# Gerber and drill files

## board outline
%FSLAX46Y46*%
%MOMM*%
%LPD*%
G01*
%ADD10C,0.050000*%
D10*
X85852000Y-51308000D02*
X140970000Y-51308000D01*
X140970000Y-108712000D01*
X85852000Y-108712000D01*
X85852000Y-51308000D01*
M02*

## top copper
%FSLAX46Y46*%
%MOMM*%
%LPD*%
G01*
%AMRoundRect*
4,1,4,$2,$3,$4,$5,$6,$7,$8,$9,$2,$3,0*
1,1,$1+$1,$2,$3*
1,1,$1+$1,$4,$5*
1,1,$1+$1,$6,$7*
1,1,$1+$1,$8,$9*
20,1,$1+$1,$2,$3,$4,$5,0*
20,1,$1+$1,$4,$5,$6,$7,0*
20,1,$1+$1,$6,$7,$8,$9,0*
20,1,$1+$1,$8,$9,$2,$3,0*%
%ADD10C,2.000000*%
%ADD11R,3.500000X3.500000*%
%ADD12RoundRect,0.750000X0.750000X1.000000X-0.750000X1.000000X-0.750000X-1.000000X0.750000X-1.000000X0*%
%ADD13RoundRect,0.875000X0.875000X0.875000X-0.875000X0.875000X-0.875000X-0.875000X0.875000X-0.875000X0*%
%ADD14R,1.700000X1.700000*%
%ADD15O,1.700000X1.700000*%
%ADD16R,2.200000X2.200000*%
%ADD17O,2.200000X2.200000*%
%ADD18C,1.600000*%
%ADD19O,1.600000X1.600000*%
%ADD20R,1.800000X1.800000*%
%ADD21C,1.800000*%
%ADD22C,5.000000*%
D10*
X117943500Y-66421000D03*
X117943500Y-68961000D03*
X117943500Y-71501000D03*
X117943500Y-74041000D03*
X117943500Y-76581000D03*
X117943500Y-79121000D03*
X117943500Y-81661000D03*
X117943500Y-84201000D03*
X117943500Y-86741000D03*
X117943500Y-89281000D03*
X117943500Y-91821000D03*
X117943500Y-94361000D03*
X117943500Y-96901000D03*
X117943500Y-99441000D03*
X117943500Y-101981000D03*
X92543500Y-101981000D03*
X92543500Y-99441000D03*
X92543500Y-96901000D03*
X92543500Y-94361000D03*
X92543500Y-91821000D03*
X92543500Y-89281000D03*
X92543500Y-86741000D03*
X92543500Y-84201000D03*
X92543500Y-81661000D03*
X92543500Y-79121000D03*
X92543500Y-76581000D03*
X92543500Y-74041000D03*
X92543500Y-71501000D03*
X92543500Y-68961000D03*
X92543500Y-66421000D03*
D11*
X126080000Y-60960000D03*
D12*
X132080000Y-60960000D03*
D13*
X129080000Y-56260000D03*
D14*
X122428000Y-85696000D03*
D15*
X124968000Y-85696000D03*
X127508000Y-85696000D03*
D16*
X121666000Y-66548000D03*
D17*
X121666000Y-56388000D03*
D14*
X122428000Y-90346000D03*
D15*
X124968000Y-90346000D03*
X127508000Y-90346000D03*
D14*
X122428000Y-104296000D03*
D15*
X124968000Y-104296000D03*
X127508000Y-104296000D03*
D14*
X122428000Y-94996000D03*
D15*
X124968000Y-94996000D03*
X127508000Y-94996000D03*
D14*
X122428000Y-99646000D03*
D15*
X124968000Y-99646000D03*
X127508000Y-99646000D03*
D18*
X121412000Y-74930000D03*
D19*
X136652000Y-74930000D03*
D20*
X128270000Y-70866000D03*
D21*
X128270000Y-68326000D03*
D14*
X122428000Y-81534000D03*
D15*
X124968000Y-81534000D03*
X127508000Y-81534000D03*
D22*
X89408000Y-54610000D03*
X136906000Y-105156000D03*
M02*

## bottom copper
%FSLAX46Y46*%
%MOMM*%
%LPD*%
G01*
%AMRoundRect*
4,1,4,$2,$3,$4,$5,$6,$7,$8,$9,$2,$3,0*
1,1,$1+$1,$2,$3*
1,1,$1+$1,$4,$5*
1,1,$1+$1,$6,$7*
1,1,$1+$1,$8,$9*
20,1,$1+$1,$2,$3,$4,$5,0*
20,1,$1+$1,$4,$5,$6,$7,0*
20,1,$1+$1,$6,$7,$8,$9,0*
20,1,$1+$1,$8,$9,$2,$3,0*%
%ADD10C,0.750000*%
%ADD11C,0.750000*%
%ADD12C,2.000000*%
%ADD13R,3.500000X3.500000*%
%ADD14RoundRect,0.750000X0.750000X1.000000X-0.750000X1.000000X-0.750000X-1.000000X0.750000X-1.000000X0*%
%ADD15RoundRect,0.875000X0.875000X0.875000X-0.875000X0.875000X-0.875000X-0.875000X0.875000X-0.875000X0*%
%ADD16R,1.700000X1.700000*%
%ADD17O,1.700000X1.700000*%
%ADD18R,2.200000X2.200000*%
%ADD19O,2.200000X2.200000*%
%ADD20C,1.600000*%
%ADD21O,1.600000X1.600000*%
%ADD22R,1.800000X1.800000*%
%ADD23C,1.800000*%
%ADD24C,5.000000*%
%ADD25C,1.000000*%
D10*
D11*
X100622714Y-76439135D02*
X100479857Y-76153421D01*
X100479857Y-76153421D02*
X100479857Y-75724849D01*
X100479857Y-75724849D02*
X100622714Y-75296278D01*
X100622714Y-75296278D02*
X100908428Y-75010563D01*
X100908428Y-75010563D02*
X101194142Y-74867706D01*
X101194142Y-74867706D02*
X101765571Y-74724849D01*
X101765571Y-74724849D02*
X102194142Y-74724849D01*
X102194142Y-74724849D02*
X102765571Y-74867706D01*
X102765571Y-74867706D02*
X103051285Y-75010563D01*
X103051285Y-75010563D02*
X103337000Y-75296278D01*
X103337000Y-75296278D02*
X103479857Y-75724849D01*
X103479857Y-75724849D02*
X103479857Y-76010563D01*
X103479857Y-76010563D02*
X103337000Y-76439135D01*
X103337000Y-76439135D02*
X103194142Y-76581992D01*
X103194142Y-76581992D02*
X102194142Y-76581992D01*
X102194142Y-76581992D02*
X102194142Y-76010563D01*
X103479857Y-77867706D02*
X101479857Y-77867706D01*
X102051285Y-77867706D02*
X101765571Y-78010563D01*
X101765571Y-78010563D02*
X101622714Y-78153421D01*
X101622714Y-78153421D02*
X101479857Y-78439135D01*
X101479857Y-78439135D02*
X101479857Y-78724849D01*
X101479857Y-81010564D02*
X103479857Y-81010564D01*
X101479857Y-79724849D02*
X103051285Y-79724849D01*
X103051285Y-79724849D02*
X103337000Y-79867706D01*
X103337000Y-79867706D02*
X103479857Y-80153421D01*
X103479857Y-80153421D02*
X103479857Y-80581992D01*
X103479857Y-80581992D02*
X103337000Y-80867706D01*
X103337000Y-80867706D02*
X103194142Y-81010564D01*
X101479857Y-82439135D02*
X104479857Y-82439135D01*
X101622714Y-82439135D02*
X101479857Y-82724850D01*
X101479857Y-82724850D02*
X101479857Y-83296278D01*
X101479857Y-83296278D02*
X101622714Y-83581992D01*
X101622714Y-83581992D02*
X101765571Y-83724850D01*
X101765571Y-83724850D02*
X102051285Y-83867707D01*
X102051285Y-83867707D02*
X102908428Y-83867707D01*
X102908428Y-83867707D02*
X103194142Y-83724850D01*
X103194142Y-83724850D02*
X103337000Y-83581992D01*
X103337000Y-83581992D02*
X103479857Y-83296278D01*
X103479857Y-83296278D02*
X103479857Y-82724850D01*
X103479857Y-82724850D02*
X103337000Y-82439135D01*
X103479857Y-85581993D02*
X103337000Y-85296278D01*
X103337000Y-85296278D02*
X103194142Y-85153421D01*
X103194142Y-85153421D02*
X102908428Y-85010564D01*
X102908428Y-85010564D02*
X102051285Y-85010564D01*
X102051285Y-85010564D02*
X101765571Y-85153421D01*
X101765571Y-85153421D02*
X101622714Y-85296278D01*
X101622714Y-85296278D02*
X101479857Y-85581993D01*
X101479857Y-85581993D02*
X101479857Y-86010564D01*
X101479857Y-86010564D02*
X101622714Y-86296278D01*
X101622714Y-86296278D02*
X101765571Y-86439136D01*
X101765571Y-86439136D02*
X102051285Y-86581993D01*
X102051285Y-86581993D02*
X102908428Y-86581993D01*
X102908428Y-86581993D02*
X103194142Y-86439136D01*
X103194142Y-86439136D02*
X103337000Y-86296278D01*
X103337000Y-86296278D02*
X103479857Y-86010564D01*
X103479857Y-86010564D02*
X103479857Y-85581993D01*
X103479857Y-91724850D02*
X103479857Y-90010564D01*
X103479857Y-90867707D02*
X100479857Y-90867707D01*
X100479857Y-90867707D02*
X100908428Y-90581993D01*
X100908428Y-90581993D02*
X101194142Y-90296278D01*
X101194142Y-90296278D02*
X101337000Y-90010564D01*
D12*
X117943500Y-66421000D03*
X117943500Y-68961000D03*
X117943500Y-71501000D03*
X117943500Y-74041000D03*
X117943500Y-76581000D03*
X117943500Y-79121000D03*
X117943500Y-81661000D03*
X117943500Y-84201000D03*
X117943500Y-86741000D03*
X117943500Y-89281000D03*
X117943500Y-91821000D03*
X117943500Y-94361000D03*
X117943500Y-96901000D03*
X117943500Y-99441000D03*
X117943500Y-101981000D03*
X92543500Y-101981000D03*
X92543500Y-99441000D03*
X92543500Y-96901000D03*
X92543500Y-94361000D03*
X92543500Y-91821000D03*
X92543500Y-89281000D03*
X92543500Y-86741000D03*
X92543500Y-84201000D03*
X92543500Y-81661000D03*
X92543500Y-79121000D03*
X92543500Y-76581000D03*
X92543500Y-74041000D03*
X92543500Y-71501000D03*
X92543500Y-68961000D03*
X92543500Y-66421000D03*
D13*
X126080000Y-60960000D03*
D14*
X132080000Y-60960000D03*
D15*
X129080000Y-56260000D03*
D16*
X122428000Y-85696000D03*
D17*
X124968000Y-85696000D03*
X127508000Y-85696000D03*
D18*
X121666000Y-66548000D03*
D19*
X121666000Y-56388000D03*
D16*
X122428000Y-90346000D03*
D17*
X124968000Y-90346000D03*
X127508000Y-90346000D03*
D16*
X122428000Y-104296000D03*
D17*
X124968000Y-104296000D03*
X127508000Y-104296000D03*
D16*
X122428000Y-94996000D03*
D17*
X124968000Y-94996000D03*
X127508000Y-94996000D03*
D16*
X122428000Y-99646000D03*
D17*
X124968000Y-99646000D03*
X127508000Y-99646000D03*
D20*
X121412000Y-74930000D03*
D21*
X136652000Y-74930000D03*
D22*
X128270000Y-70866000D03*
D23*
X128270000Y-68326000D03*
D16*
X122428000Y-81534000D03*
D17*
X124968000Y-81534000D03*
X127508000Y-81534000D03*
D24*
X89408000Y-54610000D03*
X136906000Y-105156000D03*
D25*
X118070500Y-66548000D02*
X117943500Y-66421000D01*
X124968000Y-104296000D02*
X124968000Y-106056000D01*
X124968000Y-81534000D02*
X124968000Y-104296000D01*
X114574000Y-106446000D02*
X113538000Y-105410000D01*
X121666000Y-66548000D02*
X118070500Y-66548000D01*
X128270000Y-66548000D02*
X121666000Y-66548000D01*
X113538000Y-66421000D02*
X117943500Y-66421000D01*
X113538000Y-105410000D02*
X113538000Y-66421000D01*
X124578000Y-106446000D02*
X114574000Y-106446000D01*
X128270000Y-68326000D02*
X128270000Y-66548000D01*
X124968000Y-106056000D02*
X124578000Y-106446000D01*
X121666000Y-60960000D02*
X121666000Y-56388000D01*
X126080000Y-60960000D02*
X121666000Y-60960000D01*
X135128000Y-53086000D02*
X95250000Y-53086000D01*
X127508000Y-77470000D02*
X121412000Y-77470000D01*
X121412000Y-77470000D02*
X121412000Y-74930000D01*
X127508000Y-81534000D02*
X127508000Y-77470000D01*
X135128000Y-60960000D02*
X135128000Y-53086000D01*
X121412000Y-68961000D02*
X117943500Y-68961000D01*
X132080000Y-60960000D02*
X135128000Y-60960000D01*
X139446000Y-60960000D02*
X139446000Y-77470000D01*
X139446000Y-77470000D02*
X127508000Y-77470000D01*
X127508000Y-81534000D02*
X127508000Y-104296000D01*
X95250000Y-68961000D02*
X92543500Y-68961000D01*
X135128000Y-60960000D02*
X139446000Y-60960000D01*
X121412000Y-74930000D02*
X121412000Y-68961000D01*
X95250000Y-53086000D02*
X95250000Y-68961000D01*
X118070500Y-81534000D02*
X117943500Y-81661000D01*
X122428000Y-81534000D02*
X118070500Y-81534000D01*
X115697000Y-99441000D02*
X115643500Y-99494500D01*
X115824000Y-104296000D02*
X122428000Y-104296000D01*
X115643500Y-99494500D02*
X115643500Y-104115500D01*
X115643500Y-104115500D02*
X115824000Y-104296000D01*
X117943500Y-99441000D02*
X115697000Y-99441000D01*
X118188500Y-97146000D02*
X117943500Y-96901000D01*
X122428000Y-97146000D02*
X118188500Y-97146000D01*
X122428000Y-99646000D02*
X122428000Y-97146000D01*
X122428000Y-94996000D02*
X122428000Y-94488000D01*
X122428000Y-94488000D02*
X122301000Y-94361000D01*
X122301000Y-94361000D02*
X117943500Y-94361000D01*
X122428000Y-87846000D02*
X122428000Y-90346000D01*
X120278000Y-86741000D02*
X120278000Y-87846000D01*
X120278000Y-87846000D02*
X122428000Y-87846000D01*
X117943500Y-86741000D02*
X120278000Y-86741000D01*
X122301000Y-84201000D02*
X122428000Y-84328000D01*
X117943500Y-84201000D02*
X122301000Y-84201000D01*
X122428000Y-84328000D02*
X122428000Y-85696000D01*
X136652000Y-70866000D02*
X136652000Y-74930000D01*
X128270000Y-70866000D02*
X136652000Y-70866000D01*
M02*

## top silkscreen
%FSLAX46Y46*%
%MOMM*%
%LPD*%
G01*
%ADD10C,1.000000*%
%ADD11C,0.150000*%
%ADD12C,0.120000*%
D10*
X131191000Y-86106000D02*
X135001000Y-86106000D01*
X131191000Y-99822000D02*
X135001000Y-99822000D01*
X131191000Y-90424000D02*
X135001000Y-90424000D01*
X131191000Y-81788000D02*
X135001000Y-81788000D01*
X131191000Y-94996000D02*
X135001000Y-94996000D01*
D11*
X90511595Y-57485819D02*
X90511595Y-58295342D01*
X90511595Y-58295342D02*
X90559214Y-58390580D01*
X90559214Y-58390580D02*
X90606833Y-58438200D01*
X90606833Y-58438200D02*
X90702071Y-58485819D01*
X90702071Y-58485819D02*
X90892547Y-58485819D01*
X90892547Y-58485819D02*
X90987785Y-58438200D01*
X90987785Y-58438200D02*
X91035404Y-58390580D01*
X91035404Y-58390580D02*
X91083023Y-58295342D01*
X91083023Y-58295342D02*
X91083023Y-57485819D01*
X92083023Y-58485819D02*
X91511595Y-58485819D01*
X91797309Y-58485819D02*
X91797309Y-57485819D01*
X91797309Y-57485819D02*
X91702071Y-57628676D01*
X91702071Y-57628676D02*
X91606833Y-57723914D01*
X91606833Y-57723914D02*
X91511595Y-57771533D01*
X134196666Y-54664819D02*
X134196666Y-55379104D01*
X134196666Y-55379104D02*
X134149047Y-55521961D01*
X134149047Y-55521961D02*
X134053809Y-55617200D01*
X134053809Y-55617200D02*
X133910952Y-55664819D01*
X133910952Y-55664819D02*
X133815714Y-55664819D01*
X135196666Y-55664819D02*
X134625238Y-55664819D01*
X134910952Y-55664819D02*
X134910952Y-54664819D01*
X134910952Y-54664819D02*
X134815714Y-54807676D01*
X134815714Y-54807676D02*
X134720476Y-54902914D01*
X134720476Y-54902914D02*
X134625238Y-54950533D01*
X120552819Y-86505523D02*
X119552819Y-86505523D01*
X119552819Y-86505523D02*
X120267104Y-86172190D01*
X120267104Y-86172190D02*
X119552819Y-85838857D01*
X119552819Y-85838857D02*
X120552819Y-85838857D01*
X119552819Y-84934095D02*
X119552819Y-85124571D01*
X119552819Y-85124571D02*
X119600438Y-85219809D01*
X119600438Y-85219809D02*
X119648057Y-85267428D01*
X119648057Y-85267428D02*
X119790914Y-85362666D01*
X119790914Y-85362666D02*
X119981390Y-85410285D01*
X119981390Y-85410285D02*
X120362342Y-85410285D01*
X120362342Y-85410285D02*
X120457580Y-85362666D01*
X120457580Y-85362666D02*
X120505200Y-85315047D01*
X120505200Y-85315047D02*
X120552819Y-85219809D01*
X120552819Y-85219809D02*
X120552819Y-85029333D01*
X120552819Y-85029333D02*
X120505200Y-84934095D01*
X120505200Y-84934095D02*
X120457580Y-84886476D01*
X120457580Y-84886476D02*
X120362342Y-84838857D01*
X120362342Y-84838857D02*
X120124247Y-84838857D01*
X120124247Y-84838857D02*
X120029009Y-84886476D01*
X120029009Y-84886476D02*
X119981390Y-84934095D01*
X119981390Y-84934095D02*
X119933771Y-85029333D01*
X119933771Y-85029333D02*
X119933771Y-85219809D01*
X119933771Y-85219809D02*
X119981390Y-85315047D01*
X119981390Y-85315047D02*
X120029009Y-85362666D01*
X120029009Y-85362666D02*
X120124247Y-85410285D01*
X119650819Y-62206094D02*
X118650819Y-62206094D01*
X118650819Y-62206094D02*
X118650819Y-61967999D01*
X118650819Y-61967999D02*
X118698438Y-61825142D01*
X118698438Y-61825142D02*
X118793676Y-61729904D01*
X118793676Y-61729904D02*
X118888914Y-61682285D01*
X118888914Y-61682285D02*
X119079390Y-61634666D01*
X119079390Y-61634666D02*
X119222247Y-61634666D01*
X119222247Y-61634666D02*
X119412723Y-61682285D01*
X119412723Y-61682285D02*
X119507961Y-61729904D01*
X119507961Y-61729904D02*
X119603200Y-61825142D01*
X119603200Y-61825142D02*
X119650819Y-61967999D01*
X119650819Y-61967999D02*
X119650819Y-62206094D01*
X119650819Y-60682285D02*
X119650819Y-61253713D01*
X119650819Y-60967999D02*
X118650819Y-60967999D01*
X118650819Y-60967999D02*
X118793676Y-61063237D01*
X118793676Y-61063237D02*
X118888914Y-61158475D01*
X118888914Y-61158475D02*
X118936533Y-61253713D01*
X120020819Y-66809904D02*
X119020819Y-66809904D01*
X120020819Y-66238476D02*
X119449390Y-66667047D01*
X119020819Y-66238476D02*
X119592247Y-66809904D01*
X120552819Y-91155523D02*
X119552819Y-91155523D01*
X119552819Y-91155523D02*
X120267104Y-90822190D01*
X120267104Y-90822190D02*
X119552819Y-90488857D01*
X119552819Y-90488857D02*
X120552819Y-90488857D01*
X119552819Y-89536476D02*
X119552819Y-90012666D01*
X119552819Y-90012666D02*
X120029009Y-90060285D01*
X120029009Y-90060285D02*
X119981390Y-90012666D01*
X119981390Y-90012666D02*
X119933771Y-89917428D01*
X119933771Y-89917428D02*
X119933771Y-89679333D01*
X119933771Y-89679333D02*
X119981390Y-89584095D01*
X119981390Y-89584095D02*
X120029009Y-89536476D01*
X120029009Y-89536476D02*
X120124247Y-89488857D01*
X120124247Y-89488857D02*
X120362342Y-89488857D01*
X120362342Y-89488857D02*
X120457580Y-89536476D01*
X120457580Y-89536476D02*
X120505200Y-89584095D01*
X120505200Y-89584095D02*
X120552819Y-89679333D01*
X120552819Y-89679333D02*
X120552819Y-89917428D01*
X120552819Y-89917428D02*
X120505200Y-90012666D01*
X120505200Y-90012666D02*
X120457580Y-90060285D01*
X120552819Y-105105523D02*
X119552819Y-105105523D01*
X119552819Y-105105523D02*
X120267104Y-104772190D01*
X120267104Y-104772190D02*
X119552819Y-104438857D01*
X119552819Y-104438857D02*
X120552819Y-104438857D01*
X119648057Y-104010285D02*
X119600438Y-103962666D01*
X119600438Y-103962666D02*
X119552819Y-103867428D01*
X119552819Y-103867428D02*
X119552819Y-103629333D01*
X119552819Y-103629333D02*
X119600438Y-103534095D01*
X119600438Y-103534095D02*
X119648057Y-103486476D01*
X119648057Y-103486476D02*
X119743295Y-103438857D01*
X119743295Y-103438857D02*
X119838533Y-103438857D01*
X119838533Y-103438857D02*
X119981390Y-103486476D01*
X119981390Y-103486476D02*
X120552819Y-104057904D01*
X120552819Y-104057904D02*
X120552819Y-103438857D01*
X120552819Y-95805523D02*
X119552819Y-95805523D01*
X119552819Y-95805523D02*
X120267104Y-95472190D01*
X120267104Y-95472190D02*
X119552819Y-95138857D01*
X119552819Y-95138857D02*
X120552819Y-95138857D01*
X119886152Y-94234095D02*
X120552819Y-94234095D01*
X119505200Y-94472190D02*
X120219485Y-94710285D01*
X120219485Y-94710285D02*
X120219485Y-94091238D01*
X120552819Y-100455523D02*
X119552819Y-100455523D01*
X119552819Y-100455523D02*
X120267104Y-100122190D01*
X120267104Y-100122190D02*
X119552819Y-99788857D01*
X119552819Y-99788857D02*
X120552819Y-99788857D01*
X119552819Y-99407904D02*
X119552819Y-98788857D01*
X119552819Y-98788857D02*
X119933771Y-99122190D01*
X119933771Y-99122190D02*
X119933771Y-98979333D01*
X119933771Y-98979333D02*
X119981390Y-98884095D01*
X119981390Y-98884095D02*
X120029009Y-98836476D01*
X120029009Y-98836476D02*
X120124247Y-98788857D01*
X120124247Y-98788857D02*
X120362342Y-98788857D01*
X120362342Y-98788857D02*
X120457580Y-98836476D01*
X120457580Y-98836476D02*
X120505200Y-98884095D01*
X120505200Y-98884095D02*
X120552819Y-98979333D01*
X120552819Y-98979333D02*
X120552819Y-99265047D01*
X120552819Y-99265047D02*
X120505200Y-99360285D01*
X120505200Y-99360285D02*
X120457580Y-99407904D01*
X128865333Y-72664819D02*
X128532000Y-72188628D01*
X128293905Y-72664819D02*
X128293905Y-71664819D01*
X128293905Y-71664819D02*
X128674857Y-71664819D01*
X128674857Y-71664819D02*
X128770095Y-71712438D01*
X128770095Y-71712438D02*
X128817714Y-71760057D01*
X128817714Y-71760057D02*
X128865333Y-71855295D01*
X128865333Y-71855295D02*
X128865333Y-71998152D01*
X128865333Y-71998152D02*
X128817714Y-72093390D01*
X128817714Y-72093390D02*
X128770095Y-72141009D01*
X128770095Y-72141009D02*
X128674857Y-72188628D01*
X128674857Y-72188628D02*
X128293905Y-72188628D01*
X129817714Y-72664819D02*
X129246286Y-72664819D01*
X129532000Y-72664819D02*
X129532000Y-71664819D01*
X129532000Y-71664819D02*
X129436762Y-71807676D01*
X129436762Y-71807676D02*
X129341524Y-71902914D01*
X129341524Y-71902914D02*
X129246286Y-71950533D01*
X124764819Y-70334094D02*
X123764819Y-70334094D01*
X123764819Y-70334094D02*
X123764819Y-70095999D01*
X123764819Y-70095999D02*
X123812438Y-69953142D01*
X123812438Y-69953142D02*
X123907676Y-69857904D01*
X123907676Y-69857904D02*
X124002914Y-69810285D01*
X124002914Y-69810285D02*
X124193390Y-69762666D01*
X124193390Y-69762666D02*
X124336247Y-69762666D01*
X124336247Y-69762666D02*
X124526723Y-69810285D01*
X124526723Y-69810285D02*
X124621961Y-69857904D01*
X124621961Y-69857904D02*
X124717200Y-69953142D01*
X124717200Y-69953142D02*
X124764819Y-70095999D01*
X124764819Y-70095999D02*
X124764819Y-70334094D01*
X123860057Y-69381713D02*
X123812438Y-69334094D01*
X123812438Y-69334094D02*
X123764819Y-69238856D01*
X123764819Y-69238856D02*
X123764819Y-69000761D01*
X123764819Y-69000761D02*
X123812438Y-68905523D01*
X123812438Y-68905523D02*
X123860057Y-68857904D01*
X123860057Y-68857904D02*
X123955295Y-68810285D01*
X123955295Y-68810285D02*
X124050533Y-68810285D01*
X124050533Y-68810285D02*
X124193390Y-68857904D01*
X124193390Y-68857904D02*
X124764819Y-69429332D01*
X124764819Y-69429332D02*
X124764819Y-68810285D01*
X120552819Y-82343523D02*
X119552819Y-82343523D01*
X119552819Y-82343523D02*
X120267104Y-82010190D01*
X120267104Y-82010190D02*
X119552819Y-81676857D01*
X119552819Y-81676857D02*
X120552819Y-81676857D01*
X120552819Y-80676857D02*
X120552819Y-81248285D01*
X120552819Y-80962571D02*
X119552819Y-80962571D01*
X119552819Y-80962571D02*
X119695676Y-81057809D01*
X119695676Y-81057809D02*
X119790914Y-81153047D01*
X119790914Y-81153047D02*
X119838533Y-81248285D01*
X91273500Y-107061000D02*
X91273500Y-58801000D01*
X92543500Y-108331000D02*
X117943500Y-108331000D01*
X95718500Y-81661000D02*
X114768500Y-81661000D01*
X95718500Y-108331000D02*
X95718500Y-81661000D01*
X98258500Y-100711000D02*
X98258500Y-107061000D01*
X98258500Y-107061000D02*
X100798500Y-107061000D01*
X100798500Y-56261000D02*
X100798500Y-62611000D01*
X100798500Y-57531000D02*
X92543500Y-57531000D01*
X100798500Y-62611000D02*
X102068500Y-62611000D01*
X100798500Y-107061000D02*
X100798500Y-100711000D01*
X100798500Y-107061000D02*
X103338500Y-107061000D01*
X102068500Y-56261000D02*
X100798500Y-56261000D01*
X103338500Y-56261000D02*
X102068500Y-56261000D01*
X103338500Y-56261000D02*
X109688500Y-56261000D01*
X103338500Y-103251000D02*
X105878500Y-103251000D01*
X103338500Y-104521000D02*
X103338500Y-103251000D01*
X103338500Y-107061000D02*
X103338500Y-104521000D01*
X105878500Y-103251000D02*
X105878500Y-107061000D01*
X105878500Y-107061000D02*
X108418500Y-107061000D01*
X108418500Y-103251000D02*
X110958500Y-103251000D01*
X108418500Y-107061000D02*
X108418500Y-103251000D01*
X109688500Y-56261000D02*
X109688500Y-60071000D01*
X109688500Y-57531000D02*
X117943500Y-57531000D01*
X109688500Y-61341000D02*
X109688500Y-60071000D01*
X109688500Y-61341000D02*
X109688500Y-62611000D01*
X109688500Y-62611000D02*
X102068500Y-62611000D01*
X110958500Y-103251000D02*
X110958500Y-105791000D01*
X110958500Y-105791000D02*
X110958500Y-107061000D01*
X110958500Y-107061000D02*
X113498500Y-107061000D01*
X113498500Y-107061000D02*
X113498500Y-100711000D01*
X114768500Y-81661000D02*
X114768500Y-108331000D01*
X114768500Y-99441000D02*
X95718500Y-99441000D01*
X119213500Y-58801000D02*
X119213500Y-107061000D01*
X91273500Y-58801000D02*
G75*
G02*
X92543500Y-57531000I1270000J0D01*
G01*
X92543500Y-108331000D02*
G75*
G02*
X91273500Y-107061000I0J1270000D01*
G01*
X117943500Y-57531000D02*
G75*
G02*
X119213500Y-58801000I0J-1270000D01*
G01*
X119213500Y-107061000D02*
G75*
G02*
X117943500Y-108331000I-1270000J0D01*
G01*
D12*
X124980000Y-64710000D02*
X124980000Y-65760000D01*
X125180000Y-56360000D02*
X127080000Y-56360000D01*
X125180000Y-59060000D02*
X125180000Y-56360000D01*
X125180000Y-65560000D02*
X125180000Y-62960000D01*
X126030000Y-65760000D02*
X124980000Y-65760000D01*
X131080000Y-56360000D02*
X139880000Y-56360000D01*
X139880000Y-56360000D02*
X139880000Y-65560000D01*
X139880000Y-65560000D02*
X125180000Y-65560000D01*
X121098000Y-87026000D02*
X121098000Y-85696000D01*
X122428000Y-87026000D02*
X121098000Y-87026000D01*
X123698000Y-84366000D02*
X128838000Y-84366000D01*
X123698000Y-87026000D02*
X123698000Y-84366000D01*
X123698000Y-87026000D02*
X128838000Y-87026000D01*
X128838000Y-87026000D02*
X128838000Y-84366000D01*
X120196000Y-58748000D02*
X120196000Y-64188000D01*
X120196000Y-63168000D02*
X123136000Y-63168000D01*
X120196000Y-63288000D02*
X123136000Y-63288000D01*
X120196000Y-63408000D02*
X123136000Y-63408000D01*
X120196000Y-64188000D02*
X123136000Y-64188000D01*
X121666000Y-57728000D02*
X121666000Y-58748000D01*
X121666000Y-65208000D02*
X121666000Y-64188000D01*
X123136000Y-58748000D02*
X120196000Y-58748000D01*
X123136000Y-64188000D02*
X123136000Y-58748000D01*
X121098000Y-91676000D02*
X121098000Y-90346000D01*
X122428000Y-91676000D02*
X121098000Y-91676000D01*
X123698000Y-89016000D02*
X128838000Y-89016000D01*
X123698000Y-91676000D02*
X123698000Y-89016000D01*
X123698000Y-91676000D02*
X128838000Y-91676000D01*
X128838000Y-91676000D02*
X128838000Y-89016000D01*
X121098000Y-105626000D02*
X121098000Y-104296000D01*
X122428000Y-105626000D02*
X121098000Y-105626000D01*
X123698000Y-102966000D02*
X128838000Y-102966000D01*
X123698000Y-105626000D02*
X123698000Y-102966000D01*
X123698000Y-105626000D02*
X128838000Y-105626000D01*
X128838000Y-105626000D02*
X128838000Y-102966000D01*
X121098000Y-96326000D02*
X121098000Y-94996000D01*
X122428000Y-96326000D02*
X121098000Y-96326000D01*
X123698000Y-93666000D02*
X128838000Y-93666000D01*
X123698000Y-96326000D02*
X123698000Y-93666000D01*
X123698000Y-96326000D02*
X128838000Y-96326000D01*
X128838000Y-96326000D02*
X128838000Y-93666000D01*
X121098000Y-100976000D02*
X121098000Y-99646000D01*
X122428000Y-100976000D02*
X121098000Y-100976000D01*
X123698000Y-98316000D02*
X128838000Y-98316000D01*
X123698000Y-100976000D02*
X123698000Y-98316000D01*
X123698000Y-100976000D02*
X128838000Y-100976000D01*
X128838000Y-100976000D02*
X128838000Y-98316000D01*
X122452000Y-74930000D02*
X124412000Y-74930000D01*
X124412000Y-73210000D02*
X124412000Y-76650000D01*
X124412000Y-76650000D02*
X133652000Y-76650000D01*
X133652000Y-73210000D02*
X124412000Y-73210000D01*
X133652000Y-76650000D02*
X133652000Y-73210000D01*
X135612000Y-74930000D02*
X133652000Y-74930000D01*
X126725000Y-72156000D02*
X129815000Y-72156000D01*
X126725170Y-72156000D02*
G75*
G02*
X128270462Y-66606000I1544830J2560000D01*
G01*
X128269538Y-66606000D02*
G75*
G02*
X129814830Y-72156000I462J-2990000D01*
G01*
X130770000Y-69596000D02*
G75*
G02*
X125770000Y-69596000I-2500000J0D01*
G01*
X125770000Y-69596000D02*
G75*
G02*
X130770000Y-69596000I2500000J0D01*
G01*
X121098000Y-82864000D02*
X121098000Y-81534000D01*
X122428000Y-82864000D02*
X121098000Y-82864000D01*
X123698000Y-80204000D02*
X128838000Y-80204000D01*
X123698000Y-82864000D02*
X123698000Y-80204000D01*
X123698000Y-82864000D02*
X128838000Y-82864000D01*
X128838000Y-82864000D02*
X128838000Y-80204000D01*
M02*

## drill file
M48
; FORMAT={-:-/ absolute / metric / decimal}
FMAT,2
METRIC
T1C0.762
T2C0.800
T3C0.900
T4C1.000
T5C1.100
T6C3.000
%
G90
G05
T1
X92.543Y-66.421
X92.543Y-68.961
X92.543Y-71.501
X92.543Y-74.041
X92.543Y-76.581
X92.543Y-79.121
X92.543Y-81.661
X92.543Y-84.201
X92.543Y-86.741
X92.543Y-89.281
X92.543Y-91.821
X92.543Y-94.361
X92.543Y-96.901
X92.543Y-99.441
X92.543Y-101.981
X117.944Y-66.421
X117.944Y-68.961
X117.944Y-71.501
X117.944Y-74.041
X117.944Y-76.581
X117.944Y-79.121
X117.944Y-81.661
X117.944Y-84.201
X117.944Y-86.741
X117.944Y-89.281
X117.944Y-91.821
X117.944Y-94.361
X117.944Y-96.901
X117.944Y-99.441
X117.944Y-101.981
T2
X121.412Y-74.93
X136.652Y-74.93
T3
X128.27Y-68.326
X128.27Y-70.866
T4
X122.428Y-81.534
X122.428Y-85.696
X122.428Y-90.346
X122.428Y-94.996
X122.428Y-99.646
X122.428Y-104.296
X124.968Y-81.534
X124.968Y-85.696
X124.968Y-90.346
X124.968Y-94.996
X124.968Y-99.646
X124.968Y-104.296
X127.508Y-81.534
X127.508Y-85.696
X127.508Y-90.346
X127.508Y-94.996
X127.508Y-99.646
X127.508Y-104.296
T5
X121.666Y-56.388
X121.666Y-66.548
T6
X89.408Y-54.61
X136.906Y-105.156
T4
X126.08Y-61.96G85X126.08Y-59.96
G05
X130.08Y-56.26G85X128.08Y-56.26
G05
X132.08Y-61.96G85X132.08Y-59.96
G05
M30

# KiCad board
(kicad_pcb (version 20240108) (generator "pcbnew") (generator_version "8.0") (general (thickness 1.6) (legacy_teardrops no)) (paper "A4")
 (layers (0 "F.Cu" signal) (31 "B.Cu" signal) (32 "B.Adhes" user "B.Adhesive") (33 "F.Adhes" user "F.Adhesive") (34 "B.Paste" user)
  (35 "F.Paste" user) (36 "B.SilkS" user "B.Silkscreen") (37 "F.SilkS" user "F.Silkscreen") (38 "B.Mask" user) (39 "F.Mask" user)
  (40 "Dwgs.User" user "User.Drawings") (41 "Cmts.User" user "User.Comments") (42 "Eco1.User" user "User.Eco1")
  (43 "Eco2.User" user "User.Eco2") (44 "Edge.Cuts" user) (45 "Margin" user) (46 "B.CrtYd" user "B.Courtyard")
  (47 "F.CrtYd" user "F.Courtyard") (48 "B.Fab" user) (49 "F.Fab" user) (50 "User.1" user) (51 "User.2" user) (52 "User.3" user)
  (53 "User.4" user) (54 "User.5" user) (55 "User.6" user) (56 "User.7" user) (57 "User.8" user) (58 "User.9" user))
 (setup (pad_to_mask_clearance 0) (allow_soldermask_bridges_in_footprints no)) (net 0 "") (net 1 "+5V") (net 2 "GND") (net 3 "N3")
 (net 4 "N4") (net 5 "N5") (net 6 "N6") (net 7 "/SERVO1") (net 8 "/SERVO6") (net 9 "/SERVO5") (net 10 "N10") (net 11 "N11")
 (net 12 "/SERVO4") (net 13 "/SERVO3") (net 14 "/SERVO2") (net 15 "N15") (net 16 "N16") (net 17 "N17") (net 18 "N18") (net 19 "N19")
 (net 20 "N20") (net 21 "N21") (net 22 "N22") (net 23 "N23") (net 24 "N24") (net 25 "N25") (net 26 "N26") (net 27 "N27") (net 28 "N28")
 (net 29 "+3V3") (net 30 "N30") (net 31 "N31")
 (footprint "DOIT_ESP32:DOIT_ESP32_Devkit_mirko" (layer "F.Cu") (at 91.2735 57.531)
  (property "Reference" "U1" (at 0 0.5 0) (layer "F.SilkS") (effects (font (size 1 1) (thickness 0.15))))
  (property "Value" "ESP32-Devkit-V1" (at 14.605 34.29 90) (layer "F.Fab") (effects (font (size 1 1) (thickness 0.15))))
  (fp_line (start 0 49.53) (end 0 1.27) (stroke (width 0.15) (type solid)) (layer "F.SilkS"))
  (fp_line (start 1.27 50.8) (end 26.67 50.8) (stroke (width 0.15) (type solid)) (layer "F.SilkS"))
  (fp_line (start 4.445 24.13) (end 23.495 24.13) (stroke (width 0.15) (type solid)) (layer "F.SilkS"))
  (fp_line (start 4.445 50.8) (end 4.445 24.13) (stroke (width 0.15) (type solid)) (layer "F.SilkS"))
  (fp_line (start 6.985 43.18) (end 6.985 49.53) (stroke (width 0.15) (type solid)) (layer "F.SilkS"))
  (fp_line (start 6.985 49.53) (end 9.525 49.53) (stroke (width 0.15) (type solid)) (layer "F.SilkS"))
  (fp_line (start 9.525 -1.27) (end 9.525 5.08) (stroke (width 0.15) (type solid)) (layer "F.SilkS"))
  (fp_line (start 9.525 0) (end 1.27 0) (stroke (width 0.15) (type solid)) (layer "F.SilkS"))
  (fp_line (start 9.525 5.08) (end 10.795 5.08) (stroke (width 0.15) (type solid)) (layer "F.SilkS"))
  (fp_line (start 9.525 49.53) (end 9.525 43.18) (stroke (width 0.15) (type solid)) (layer "F.SilkS"))
  (fp_line (start 9.525 49.53) (end 12.065 49.53) (stroke (width 0.15) (type solid)) (layer "F.SilkS"))
  (fp_line (start 10.795 -1.27) (end 9.525 -1.27) (stroke (width 0.15) (type solid)) (layer "F.SilkS"))
  (fp_line (start 12.065 -1.27) (end 10.795 -1.27) (stroke (width 0.15) (type solid)) (layer "F.SilkS"))
  (fp_line (start 12.065 -1.27) (end 18.415 -1.27) (stroke (width 0.15) (type solid)) (layer "F.SilkS"))
  (fp_line (start 12.065 45.72) (end 14.605 45.72) (stroke (width 0.15) (type solid)) (layer "F.SilkS"))
  (fp_line (start 12.065 46.99) (end 12.065 45.72) (stroke (width 0.15) (type solid)) (layer "F.SilkS"))
  (fp_line (start 12.065 49.53) (end 12.065 46.99) (stroke (width 0.15) (type solid)) (layer "F.SilkS"))
  (fp_line (start 14.605 45.72) (end 14.605 49.53) (stroke (width 0.15) (type solid)) (layer "F.SilkS"))
  (fp_line (start 14.605 49.53) (end 17.145 49.53) (stroke (width 0.15) (type solid)) (layer "F.SilkS"))
  (fp_line (start 17.145 45.72) (end 19.685 45.72) (stroke (width 0.15) (type solid)) (layer "F.SilkS"))
  (fp_line (start 17.145 49.53) (end 17.145 45.72) (stroke (width 0.15) (type solid)) (layer "F.SilkS"))
  (fp_line (start 18.415 -1.27) (end 18.415 2.54) (stroke (width 0.15) (type solid)) (layer "F.SilkS"))
  (fp_line (start 18.415 0) (end 26.67 0) (stroke (width 0.15) (type solid)) (layer "F.SilkS"))
  (fp_line (start 18.415 3.81) (end 18.415 2.54) (stroke (width 0.15) (type solid)) (layer "F.SilkS"))
  (fp_line (start 18.415 3.81) (end 18.415 5.08) (stroke (width 0.15) (type solid)) (layer "F.SilkS"))
  (fp_line (start 18.415 5.08) (end 10.795 5.08) (stroke (width 0.15) (type solid)) (layer "F.SilkS"))
  (fp_line (start 19.685 45.72) (end 19.685 48.26) (stroke (width 0.15) (type solid)) (layer "F.SilkS"))
  (fp_line (start 19.685 48.26) (end 19.685 49.53) (stroke (width 0.15) (type solid)) (layer "F.SilkS"))
  (fp_line (start 19.685 49.53) (end 22.225 49.53) (stroke (width 0.15) (type solid)) (layer "F.SilkS"))
  (fp_line (start 22.225 49.53) (end 22.225 43.18) (stroke (width 0.15) (type solid)) (layer "F.SilkS"))
  (fp_line (start 23.495 24.13) (end 23.495 50.8) (stroke (width 0.15) (type solid)) (layer "F.SilkS"))
  (fp_line (start 23.495 41.91) (end 4.445 41.91) (stroke (width 0.15) (type solid)) (layer "F.SilkS"))
  (fp_line (start 27.94 1.27) (end 27.94 49.53) (stroke (width 0.15) (type solid)) (layer "F.SilkS"))
  (fp_arc (start 0 1.27) (mid 0.371974 0.371974) (end 1.27 0) (stroke (width 0.15) (type solid)) (layer "F.SilkS"))
  (fp_arc (start 1.27 50.8) (mid 0.371974 50.428026) (end 0 49.53) (stroke (width 0.15) (type solid)) (layer "F.SilkS"))
  (fp_arc (start 26.67 0) (mid 27.568026 0.371974) (end 27.94 1.27) (stroke (width 0.15) (type solid)) (layer "F.SilkS"))
  (fp_arc (start 27.94 49.53) (mid 27.568026 50.428026) (end 26.67 50.8) (stroke (width 0.15) (type solid)) (layer "F.SilkS"))
  (pad "1" thru_hole circle (at 26.67 8.89) (size 2 2) (drill 0.762) (layers "*.Cu" "*.Mask") (remove_unused_layers no) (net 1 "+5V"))
  (pad "2" thru_hole circle (at 26.67 11.43) (size 2 2) (drill 0.762) (layers "*.Cu" "*.Mask") (remove_unused_layers no) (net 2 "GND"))
  (pad "3" thru_hole circle (at 26.67 13.97) (size 2 2) (drill 0.762) (layers "*.Cu" "*.Mask") (remove_unused_layers no) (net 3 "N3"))
  (pad "4" thru_hole circle (at 26.67 16.51) (size 2 2) (drill 0.762) (layers "*.Cu" "*.Mask") (remove_unused_layers no) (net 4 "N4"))
  (pad "5" thru_hole circle (at 26.67 19.05) (size 2 2) (drill 0.762) (layers "*.Cu" "*.Mask") (remove_unused_layers no) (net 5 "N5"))
  (pad "6" thru_hole circle (at 26.67 21.59) (size 2 2) (drill 0.762) (layers "*.Cu" "*.Mask") (remove_unused_layers no) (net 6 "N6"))
  (pad "7" thru_hole circle (at 26.67 24.13) (size 2 2) (drill 0.762) (layers "*.Cu" "*.Mask") (remove_unused_layers no) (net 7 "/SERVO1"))
  (pad "8" thru_hole circle (at 26.67 26.67) (size 2 2) (drill 0.762) (layers "*.Cu" "*.Mask") (remove_unused_layers no) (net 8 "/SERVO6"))
  (pad "9" thru_hole circle (at 26.67 29.21) (size 2 2) (drill 0.762) (layers "*.Cu" "*.Mask") (remove_unused_layers no) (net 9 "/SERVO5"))
  (pad "10" thru_hole circle (at 26.67 31.75) (size 2 2) (drill 0.762) (layers "*.Cu" "*.Mask") (remove_unused_layers no) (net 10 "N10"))
  (pad "11" thru_hole circle (at 26.67 34.29) (size 2 2) (drill 0.762) (layers "*.Cu" "*.Mask") (remove_unused_layers no) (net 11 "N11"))
  (pad "12" thru_hole circle (at 26.67 36.83) (size 2 2) (drill 0.762) (layers "*.Cu" "*.Mask") (remove_unused_layers no) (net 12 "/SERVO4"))
  (pad "13" thru_hole circle (at 26.67 39.37) (size 2 2) (drill 0.762) (layers "*.Cu" "*.Mask") (remove_unused_layers no) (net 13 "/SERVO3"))
  (pad "14" thru_hole circle (at 26.67 41.91) (size 2 2) (drill 0.762) (layers "*.Cu" "*.Mask") (remove_unused_layers no) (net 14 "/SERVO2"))
  (pad "15" thru_hole circle (at 26.67 44.45) (size 2 2) (drill 0.762) (layers "*.Cu" "*.Mask") (remove_unused_layers no) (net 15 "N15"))
  (pad "16" thru_hole circle (at 1.27 44.45) (size 2 2) (drill 0.762) (layers "*.Cu" "*.Mask") (remove_unused_layers no) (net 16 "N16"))
  (pad "17" thru_hole circle (at 1.27 41.91) (size 2 2) (drill 0.762) (layers "*.Cu" "*.Mask") (remove_unused_layers no) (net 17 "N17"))
  (pad "18" thru_hole circle (at 1.27 39.37) (size 2 2) (drill 0.762) (layers "*.Cu" "*.Mask") (remove_unused_layers no) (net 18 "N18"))
  (pad "19" thru_hole circle (at 1.27 36.83) (size 2 2) (drill 0.762) (layers "*.Cu" "*.Mask") (remove_unused_layers no) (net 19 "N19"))
  (pad "20" thru_hole circle (at 1.27 34.29) (size 2 2) (drill 0.762) (layers "*.Cu" "*.Mask") (remove_unused_layers no) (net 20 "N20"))
  (pad "21" thru_hole circle (at 1.27 31.75) (size 2 2) (drill 0.762) (layers "*.Cu" "*.Mask") (remove_unused_layers no) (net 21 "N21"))
  (pad "22" thru_hole circle (at 1.27 29.21) (size 2 2) (drill 0.762) (layers "*.Cu" "*.Mask") (remove_unused_layers no) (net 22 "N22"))
  (pad "23" thru_hole circle (at 1.27 26.67) (size 2 2) (drill 0.762) (layers "*.Cu" "*.Mask") (remove_unused_layers no) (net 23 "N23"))
  (pad "24" thru_hole circle (at 1.27 24.13) (size 2 2) (drill 0.762) (layers "*.Cu" "*.Mask") (remove_unused_layers no) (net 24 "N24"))
  (pad "25" thru_hole circle (at 1.27 21.59) (size 2 2) (drill 0.762) (layers "*.Cu" "*.Mask") (remove_unused_layers no) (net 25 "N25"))
  (pad "26" thru_hole circle (at 1.27 19.05) (size 2 2) (drill 0.762) (layers "*.Cu" "*.Mask") (remove_unused_layers no) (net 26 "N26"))
  (pad "27" thru_hole circle (at 1.27 16.51) (size 2 2) (drill 0.762) (layers "*.Cu" "*.Mask") (remove_unused_layers no) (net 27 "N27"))
  (pad "28" thru_hole circle (at 1.27 13.97) (size 2 2) (drill 0.762) (layers "*.Cu" "*.Mask") (remove_unused_layers no) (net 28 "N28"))
  (pad "29" thru_hole circle (at 1.27 11.43) (size 2 2) (drill 0.762) (layers "*.Cu" "*.Mask") (remove_unused_layers no) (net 2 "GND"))
  (pad "30" thru_hole circle (at 1.27 8.89) (size 2 2) (drill 0.762) (layers "*.Cu" "*.Mask") (remove_unused_layers no) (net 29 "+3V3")))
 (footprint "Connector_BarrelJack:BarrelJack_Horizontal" (layer "F.Cu") (at 126.08 60.96 180)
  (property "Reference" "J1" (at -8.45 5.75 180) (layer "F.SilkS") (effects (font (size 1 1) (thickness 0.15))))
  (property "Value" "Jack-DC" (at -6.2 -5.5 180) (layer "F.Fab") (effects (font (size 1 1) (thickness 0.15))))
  (fp_line (start 1.1 -3.75) (end 1.1 -4.8) (stroke (width 0.12) (type solid)) (layer "F.SilkS"))
  (fp_line (start 0.9 4.6) (end -1 4.6) (stroke (width 0.12) (type solid)) (layer "F.SilkS"))
  (fp_line (start 0.9 1.9) (end 0.9 4.6) (stroke (width 0.12) (type solid)) (layer "F.SilkS"))
  (fp_line (start 0.9 -4.6) (end 0.9 -2) (stroke (width 0.12) (type solid)) (layer "F.SilkS"))
  (fp_line (start 0.05 -4.8) (end 1.1 -4.8) (stroke (width 0.12) (type solid)) (layer "F.SilkS"))
  (fp_line (start -5 4.6) (end -13.8 4.6) (stroke (width 0.12) (type solid)) (layer "F.SilkS"))
  (fp_line (start -13.8 4.6) (end -13.8 -4.6) (stroke (width 0.12) (type solid)) (layer "F.SilkS"))
  (fp_line (start -13.8 -4.6) (end 0.9 -4.6) (stroke (width 0.12) (type solid)) (layer "F.SilkS"))
  (pad "1" thru_hole rect (at 0 0 180) (size 3.5 3.5) (drill oval 1 3) (layers "*.Cu" "*.Mask") (remove_unused_layers no) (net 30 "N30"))
  (pad "2" thru_hole roundrect (at -6 0 180) (size 3 3.5) (drill oval 1 3) (layers "*.Cu" "*.Mask") (remove_unused_layers no)
   (roundrect_rratio 0.25) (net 2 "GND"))
  (pad "3" thru_hole roundrect (at -3 4.7 180) (size 3.5 3.5) (drill oval 3 1) (layers "*.Cu" "*.Mask") (remove_unused_layers no)
   (roundrect_rratio 0.25)))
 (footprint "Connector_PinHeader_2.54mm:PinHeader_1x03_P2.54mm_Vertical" (layer "F.Cu") (at 122.428 85.696 90)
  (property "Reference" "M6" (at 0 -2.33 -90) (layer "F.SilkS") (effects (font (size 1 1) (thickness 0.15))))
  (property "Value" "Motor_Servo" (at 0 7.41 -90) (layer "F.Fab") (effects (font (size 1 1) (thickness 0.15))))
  (fp_line (start -1.33 -1.33) (end 0 -1.33) (stroke (width 0.12) (type solid)) (layer "F.SilkS"))
  (fp_line (start -1.33 0) (end -1.33 -1.33) (stroke (width 0.12) (type solid)) (layer "F.SilkS"))
  (fp_line (start 1.33 1.27) (end 1.33 6.41) (stroke (width 0.12) (type solid)) (layer "F.SilkS"))
  (fp_line (start -1.33 1.27) (end 1.33 1.27) (stroke (width 0.12) (type solid)) (layer "F.SilkS"))
  (fp_line (start -1.33 1.27) (end -1.33 6.41) (stroke (width 0.12) (type solid)) (layer "F.SilkS"))
  (fp_line (start -1.33 6.41) (end 1.33 6.41) (stroke (width 0.12) (type solid)) (layer "F.SilkS"))
  (pad "1" thru_hole rect (at 0 0 90) (size 1.7 1.7) (drill 1) (layers "*.Cu" "*.Mask") (remove_unused_layers no) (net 8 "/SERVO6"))
  (pad "2" thru_hole oval (at 0 2.54 90) (size 1.7 1.7) (drill 1) (layers "*.Cu" "*.Mask") (remove_unused_layers no) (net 1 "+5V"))
  (pad "3" thru_hole oval (at 0 5.08 90) (size 1.7 1.7) (drill 1) (layers "*.Cu" "*.Mask") (remove_unused_layers no) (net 2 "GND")))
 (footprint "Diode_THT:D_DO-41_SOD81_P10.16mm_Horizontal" (layer "F.Cu") (at 121.666 66.548 90)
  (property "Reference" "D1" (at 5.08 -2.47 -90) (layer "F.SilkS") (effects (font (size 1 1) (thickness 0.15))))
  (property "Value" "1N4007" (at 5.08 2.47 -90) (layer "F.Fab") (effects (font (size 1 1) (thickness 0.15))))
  (fp_line (start 7.8 -1.47) (end 2.36 -1.47) (stroke (width 0.12) (type solid)) (layer "F.SilkS"))
  (fp_line (start 3.38 -1.47) (end 3.38 1.47) (stroke (width 0.12) (type solid)) (layer "F.SilkS"))
  (fp_line (start 3.26 -1.47) (end 3.26 1.47) (stroke (width 0.12) (type solid)) (layer "F.SilkS"))
  (fp_line (start 3.14 -1.47) (end 3.14 1.47) (stroke (width 0.12) (type solid)) (layer "F.SilkS"))
  (fp_line (start 2.36 -1.47) (end 2.36 1.47) (stroke (width 0.12) (type solid)) (layer "F.SilkS"))
  (fp_line (start 8.82 0) (end 7.8 0) (stroke (width 0.12) (type solid)) (layer "F.SilkS"))
  (fp_line (start 1.34 0) (end 2.36 0) (stroke (width 0.12) (type solid)) (layer "F.SilkS"))
  (fp_line (start 7.8 1.47) (end 7.8 -1.47) (stroke (width 0.12) (type solid)) (layer "F.SilkS"))
  (fp_line (start 2.36 1.47) (end 7.8 1.47) (stroke (width 0.12) (type solid)) (layer "F.SilkS"))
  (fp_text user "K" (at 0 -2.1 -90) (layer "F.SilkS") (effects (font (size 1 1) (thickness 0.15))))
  (pad "1" thru_hole rect (at 0 0 90) (size 2.2 2.2) (drill 1.1) (layers "*.Cu" "*.Mask") (remove_unused_layers no) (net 1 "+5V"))
  (pad "2" thru_hole oval (at 10.16 0 90) (size 2.2 2.2) (drill 1.1) (layers "*.Cu" "*.Mask") (remove_unused_layers no) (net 30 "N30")))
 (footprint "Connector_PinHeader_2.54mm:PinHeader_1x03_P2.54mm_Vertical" (layer "F.Cu") (at 122.428 90.346 90)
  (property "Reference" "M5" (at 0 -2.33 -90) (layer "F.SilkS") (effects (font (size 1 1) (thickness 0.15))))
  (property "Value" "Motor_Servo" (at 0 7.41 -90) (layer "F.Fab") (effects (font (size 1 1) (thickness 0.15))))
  (fp_line (start -1.33 -1.33) (end 0 -1.33) (stroke (width 0.12) (type solid)) (layer "F.SilkS"))
  (fp_line (start -1.33 0) (end -1.33 -1.33) (stroke (width 0.12) (type solid)) (layer "F.SilkS"))
  (fp_line (start 1.33 1.27) (end 1.33 6.41) (stroke (width 0.12) (type solid)) (layer "F.SilkS"))
  (fp_line (start -1.33 1.27) (end 1.33 1.27) (stroke (width 0.12) (type solid)) (layer "F.SilkS"))
  (fp_line (start -1.33 1.27) (end -1.33 6.41) (stroke (width 0.12) (type solid)) (layer "F.SilkS"))
  (fp_line (start -1.33 6.41) (end 1.33 6.41) (stroke (width 0.12) (type solid)) (layer "F.SilkS"))
  (pad "1" thru_hole rect (at 0 0 90) (size 1.7 1.7) (drill 1) (layers "*.Cu" "*.Mask") (remove_unused_layers no) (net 9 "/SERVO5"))
  (pad "2" thru_hole oval (at 0 2.54 90) (size 1.7 1.7) (drill 1) (layers "*.Cu" "*.Mask") (remove_unused_layers no) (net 1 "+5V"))
  (pad "3" thru_hole oval (at 0 5.08 90) (size 1.7 1.7) (drill 1) (layers "*.Cu" "*.Mask") (remove_unused_layers no) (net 2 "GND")))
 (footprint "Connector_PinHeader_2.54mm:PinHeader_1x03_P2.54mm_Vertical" (layer "F.Cu") (at 122.428 104.296 90)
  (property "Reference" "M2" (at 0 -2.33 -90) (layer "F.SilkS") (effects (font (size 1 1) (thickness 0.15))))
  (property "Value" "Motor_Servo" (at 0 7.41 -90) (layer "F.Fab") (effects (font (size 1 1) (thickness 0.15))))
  (fp_line (start -1.33 -1.33) (end 0 -1.33) (stroke (width 0.12) (type solid)) (layer "F.SilkS"))
  (fp_line (start -1.33 0) (end -1.33 -1.33) (stroke (width 0.12) (type solid)) (layer "F.SilkS"))
  (fp_line (start 1.33 1.27) (end 1.33 6.41) (stroke (width 0.12) (type solid)) (layer "F.SilkS"))
  (fp_line (start -1.33 1.27) (end 1.33 1.27) (stroke (width 0.12) (type solid)) (layer "F.SilkS"))
  (fp_line (start -1.33 1.27) (end -1.33 6.41) (stroke (width 0.12) (type solid)) (layer "F.SilkS"))
  (fp_line (start -1.33 6.41) (end 1.33 6.41) (stroke (width 0.12) (type solid)) (layer "F.SilkS"))
  (pad "1" thru_hole rect (at 0 0 90) (size 1.7 1.7) (drill 1) (layers "*.Cu" "*.Mask") (remove_unused_layers no) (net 14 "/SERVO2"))
  (pad "2" thru_hole oval (at 0 2.54 90) (size 1.7 1.7) (drill 1) (layers "*.Cu" "*.Mask") (remove_unused_layers no) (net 1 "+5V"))
  (pad "3" thru_hole oval (at 0 5.08 90) (size 1.7 1.7) (drill 1) (layers "*.Cu" "*.Mask") (remove_unused_layers no) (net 2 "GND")))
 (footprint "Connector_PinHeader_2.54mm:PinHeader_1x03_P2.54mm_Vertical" (layer "F.Cu") (at 122.428 94.996 90)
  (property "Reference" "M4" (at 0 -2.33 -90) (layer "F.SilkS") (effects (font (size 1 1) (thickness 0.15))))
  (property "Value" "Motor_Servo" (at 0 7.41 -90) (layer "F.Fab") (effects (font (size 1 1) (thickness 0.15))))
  (fp_line (start -1.33 -1.33) (end 0 -1.33) (stroke (width 0.12) (type solid)) (layer "F.SilkS"))
  (fp_line (start -1.33 0) (end -1.33 -1.33) (stroke (width 0.12) (type solid)) (layer "F.SilkS"))
  (fp_line (start 1.33 1.27) (end 1.33 6.41) (stroke (width 0.12) (type solid)) (layer "F.SilkS"))
  (fp_line (start -1.33 1.27) (end 1.33 1.27) (stroke (width 0.12) (type solid)) (layer "F.SilkS"))
  (fp_line (start -1.33 1.27) (end -1.33 6.41) (stroke (width 0.12) (type solid)) (layer "F.SilkS"))
  (fp_line (start -1.33 6.41) (end 1.33 6.41) (stroke (width 0.12) (type solid)) (layer "F.SilkS"))
  (pad "1" thru_hole rect (at 0 0 90) (size 1.7 1.7) (drill 1) (layers "*.Cu" "*.Mask") (remove_unused_layers no) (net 12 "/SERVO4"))
  (pad "2" thru_hole oval (at 0 2.54 90) (size 1.7 1.7) (drill 1) (layers "*.Cu" "*.Mask") (remove_unused_layers no) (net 1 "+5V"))
  (pad "3" thru_hole oval (at 0 5.08 90) (size 1.7 1.7) (drill 1) (layers "*.Cu" "*.Mask") (remove_unused_layers no) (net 2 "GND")))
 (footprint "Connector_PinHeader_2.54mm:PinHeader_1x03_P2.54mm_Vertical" (layer "F.Cu") (at 122.428 99.646 90)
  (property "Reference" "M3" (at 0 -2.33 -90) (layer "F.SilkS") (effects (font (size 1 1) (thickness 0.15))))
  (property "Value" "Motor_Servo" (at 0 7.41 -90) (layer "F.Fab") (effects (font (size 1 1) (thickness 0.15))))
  (fp_line (start -1.33 -1.33) (end 0 -1.33) (stroke (width 0.12) (type solid)) (layer "F.SilkS"))
  (fp_line (start -1.33 0) (end -1.33 -1.33) (stroke (width 0.12) (type solid)) (layer "F.SilkS"))
  (fp_line (start 1.33 1.27) (end 1.33 6.41) (stroke (width 0.12) (type solid)) (layer "F.SilkS"))
  (fp_line (start -1.33 1.27) (end 1.33 1.27) (stroke (width 0.12) (type solid)) (layer "F.SilkS"))
  (fp_line (start -1.33 1.27) (end -1.33 6.41) (stroke (width 0.12) (type solid)) (layer "F.SilkS"))
  (fp_line (start -1.33 6.41) (end 1.33 6.41) (stroke (width 0.12) (type solid)) (layer "F.SilkS"))
  (pad "1" thru_hole rect (at 0 0 90) (size 1.7 1.7) (drill 1) (layers "*.Cu" "*.Mask") (remove_unused_layers no) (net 13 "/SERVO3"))
  (pad "2" thru_hole oval (at 0 2.54 90) (size 1.7 1.7) (drill 1) (layers "*.Cu" "*.Mask") (remove_unused_layers no) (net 1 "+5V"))
  (pad "3" thru_hole oval (at 0 5.08 90) (size 1.7 1.7) (drill 1) (layers "*.Cu" "*.Mask") (remove_unused_layers no) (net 2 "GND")))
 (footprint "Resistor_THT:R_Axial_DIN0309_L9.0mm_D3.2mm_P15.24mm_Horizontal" (layer "F.Cu") (at 121.412 74.93)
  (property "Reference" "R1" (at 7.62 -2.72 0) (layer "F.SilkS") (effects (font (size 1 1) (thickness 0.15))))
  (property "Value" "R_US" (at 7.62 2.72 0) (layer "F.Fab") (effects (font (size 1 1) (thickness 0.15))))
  (fp_line (start 1.04 0) (end 3 0) (stroke (width 0.12) (type solid)) (layer "F.SilkS"))
  (fp_line (start 3 -1.72) (end 3 1.72) (stroke (width 0.12) (type solid)) (layer "F.SilkS"))
  (fp_line (start 3 1.72) (end 12.24 1.72) (stroke (width 0.12) (type solid)) (layer "F.SilkS"))
  (fp_line (start 12.24 -1.72) (end 3 -1.72) (stroke (width 0.12) (type solid)) (layer "F.SilkS"))
  (fp_line (start 12.24 1.72) (end 12.24 -1.72) (stroke (width 0.12) (type solid)) (layer "F.SilkS"))
  (fp_line (start 14.2 0) (end 12.24 0) (stroke (width 0.12) (type solid)) (layer "F.SilkS"))
  (pad "1" thru_hole circle (at 0 0) (size 1.6 1.6) (drill 0.8) (layers "*.Cu" "*.Mask") (remove_unused_layers no) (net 2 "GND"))
  (pad "2" thru_hole oval (at 15.24 0) (size 1.6 1.6) (drill 0.8) (layers "*.Cu" "*.Mask") (remove_unused_layers no) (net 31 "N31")))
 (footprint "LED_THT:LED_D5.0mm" (layer "F.Cu") (at 128.27 70.866 90)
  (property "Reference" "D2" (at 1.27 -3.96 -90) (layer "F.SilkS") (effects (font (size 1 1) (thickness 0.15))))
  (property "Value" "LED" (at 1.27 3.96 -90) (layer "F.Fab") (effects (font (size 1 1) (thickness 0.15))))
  (fp_line (start -1.29 -1.545) (end -1.29 1.545) (stroke (width 0.12) (type solid)) (layer "F.SilkS"))
  (fp_arc (start -1.29 -1.54483) (mid 2.072002 -2.880433) (end 4.26 0.000462) (stroke (width 0.12) (type solid)) (layer "F.SilkS"))
  (fp_arc (start 4.26 -0.000462) (mid 2.072002 2.880433) (end -1.29 1.54483) (stroke (width 0.12) (type solid)) (layer "F.SilkS"))
  (fp_circle (center 1.27 0) (end 3.77 0) (stroke (width 0.12) (type solid)) (fill none) (layer "F.SilkS"))
  (pad "1" thru_hole rect (at 0 0 90) (size 1.8 1.8) (drill 0.9) (layers "*.Cu" "*.Mask") (remove_unused_layers no) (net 31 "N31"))
  (pad "2" thru_hole circle (at 2.54 0 90) (size 1.8 1.8) (drill 0.9) (layers "*.Cu" "*.Mask") (remove_unused_layers no) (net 1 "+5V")))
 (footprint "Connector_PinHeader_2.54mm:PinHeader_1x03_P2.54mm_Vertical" (layer "F.Cu") (at 122.428 81.534 90)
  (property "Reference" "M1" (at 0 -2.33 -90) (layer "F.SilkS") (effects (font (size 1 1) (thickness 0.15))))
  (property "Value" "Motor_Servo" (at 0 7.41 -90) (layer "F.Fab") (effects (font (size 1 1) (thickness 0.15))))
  (fp_line (start -1.33 -1.33) (end 0 -1.33) (stroke (width 0.12) (type solid)) (layer "F.SilkS"))
  (fp_line (start -1.33 0) (end -1.33 -1.33) (stroke (width 0.12) (type solid)) (layer "F.SilkS"))
  (fp_line (start 1.33 1.27) (end 1.33 6.41) (stroke (width 0.12) (type solid)) (layer "F.SilkS"))
  (fp_line (start -1.33 1.27) (end 1.33 1.27) (stroke (width 0.12) (type solid)) (layer "F.SilkS"))
  (fp_line (start -1.33 1.27) (end -1.33 6.41) (stroke (width 0.12) (type solid)) (layer "F.SilkS"))
  (fp_line (start -1.33 6.41) (end 1.33 6.41) (stroke (width 0.12) (type solid)) (layer "F.SilkS"))
  (pad "1" thru_hole rect (at 0 0 90) (size 1.7 1.7) (drill 1) (layers "*.Cu" "*.Mask") (remove_unused_layers no) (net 7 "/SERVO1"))
  (pad "2" thru_hole oval (at 0 2.54 90) (size 1.7 1.7) (drill 1) (layers "*.Cu" "*.Mask") (remove_unused_layers no) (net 1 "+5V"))
  (pad "3" thru_hole oval (at 0 5.08 90) (size 1.7 1.7) (drill 1) (layers "*.Cu" "*.Mask") (remove_unused_layers no) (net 2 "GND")))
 (gr_line (start 131.191 86.106) (end 135.001 86.106) (stroke (width 1) (type default)) (layer "F.SilkS"))
 (gr_line (start 131.191 99.822) (end 135.001 99.822) (stroke (width 1) (type default)) (layer "F.SilkS"))
 (gr_line (start 131.191 90.424) (end 135.001 90.424) (stroke (width 1) (type default)) (layer "F.SilkS"))
 (gr_line (start 131.191 81.788) (end 135.001 81.788) (stroke (width 1) (type default)) (layer "F.SilkS"))
 (gr_line (start 131.191 94.996) (end 135.001 94.996) (stroke (width 1) (type default)) (layer "F.SilkS"))
 (gr_rect (start 85.852 51.308) (end 140.97 108.712) (stroke (width 0.05) (type default)) (fill none) (layer "Edge.Cuts"))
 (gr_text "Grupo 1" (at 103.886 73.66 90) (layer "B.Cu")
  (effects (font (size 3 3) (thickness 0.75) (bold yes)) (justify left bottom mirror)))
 (via (at 89.408 54.61) (size 5) (drill 3) (layers "F.Cu" "B.Cu") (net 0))
 (via (at 136.906 105.156) (size 5) (drill 3) (layers "F.Cu" "B.Cu") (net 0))
 (segment (start 118.0705 66.548) (end 117.9435 66.421) (width 1) (layer "B.Cu") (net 1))
 (segment (start 124.968 104.296) (end 124.968 106.056) (width 1) (layer "B.Cu") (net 1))
 (segment (start 124.968 81.534) (end 124.968 104.296) (width 1) (layer "B.Cu") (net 1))
 (segment (start 114.574 106.446) (end 113.538 105.41) (width 1) (layer "B.Cu") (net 1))
 (segment (start 121.666 66.548) (end 118.0705 66.548) (width 1) (layer "B.Cu") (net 1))
 (segment (start 128.27 66.548) (end 121.666 66.548) (width 1) (layer "B.Cu") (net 1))
 (segment (start 113.538 66.421) (end 117.9435 66.421) (width 1) (layer "B.Cu") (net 1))
 (segment (start 113.538 105.41) (end 113.538 66.421) (width 1) (layer "B.Cu") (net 1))
 (segment (start 124.578 106.446) (end 114.574 106.446) (width 1) (layer "B.Cu") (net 1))
 (segment (start 128.27 68.326) (end 128.27 66.548) (width 1) (layer "B.Cu") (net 1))
 (segment (start 124.968 106.056) (end 124.578 106.446) (width 1) (layer "B.Cu") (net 1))
 (segment (start 121.666 60.96) (end 121.666 56.388) (width 1) (layer "B.Cu") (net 30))
 (segment (start 126.08 60.96) (end 121.666 60.96) (width 1) (layer "B.Cu") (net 30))
 (segment (start 135.128 53.086) (end 95.25 53.086) (width 1) (layer "B.Cu") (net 2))
 (segment (start 127.508 77.47) (end 121.412 77.47) (width 1) (layer "B.Cu") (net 2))
 (segment (start 121.412 77.47) (end 121.412 74.93) (width 1) (layer "B.Cu") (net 2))
 (segment (start 127.508 81.534) (end 127.508 77.47) (width 1) (layer "B.Cu") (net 2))
 (segment (start 135.128 60.96) (end 135.128 53.086) (width 1) (layer "B.Cu") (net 2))
 (segment (start 121.412 68.961) (end 117.9435 68.961) (width 1) (layer "B.Cu") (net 2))
 (segment (start 132.08 60.96) (end 135.128 60.96) (width 1) (layer "B.Cu") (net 2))
 (segment (start 139.446 60.96) (end 139.446 77.47) (width 1) (layer "B.Cu") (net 2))
 (segment (start 139.446 77.47) (end 127.508 77.47) (width 1) (layer "B.Cu") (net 2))
 (segment (start 127.508 81.534) (end 127.508 104.296) (width 1) (layer "B.Cu") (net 2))
 (segment (start 95.25 68.961) (end 92.5435 68.961) (width 1) (layer "B.Cu") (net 2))
 (segment (start 135.128 60.96) (end 139.446 60.96) (width 1) (layer "B.Cu") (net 2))
 (segment (start 121.412 74.93) (end 121.412 68.961) (width 1) (layer "B.Cu") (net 2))
 (segment (start 95.25 53.086) (end 95.25 68.961) (width 1) (layer "B.Cu") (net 2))
 (segment (start 118.0705 81.534) (end 117.9435 81.661) (width 1) (layer "B.Cu") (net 7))
 (segment (start 122.428 81.534) (end 118.0705 81.534) (width 1) (layer "B.Cu") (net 7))
 (segment (start 115.697 99.441) (end 115.6435 99.4945) (width 1) (layer "B.Cu") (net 14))
 (segment (start 115.824 104.296) (end 122.428 104.296) (width 1) (layer "B.Cu") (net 14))
 (segment (start 115.6435 99.4945) (end 115.6435 104.1155) (width 1) (layer "B.Cu") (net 14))
 (segment (start 115.6435 104.1155) (end 115.824 104.296) (width 1) (layer "B.Cu") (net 14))
 (segment (start 117.9435 99.441) (end 115.697 99.441) (width 1) (layer "B.Cu") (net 14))
 (segment (start 118.1885 97.146) (end 117.9435 96.901) (width 1) (layer "B.Cu") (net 13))
 (segment (start 122.428 97.146) (end 118.1885 97.146) (width 1) (layer "B.Cu") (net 13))
 (segment (start 122.428 99.646) (end 122.428 97.146) (width 1) (layer "B.Cu") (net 13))
 (segment (start 122.428 94.996) (end 122.428 94.488) (width 1) (layer "B.Cu") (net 12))
 (segment (start 122.428 94.488) (end 122.301 94.361) (width 1) (layer "B.Cu") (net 12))
 (segment (start 122.301 94.361) (end 117.9435 94.361) (width 1) (layer "B.Cu") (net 12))
 (segment (start 122.428 87.846) (end 122.428 90.346) (width 1) (layer "B.Cu") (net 9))
 (segment (start 120.278 86.741) (end 120.278 87.846) (width 1) (layer "B.Cu") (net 9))
 (segment (start 120.278 87.846) (end 122.428 87.846) (width 1) (layer "B.Cu") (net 9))
 (segment (start 117.9435 86.741) (end 120.278 86.741) (width 1) (layer "B.Cu") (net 9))
 (segment (start 122.301 84.201) (end 122.428 84.328) (width 1) (layer "B.Cu") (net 8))
 (segment (start 117.9435 84.201) (end 122.301 84.201) (width 1) (layer "B.Cu") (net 8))
 (segment (start 122.428 84.328) (end 122.428 85.696) (width 1) (layer "B.Cu") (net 8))
 (segment (start 136.652 70.866) (end 136.652 74.93) (width 1) (layer "B.Cu") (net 31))
 (segment (start 128.27 70.866) (end 136.652 70.866) (width 1) (layer "B.Cu") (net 31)))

